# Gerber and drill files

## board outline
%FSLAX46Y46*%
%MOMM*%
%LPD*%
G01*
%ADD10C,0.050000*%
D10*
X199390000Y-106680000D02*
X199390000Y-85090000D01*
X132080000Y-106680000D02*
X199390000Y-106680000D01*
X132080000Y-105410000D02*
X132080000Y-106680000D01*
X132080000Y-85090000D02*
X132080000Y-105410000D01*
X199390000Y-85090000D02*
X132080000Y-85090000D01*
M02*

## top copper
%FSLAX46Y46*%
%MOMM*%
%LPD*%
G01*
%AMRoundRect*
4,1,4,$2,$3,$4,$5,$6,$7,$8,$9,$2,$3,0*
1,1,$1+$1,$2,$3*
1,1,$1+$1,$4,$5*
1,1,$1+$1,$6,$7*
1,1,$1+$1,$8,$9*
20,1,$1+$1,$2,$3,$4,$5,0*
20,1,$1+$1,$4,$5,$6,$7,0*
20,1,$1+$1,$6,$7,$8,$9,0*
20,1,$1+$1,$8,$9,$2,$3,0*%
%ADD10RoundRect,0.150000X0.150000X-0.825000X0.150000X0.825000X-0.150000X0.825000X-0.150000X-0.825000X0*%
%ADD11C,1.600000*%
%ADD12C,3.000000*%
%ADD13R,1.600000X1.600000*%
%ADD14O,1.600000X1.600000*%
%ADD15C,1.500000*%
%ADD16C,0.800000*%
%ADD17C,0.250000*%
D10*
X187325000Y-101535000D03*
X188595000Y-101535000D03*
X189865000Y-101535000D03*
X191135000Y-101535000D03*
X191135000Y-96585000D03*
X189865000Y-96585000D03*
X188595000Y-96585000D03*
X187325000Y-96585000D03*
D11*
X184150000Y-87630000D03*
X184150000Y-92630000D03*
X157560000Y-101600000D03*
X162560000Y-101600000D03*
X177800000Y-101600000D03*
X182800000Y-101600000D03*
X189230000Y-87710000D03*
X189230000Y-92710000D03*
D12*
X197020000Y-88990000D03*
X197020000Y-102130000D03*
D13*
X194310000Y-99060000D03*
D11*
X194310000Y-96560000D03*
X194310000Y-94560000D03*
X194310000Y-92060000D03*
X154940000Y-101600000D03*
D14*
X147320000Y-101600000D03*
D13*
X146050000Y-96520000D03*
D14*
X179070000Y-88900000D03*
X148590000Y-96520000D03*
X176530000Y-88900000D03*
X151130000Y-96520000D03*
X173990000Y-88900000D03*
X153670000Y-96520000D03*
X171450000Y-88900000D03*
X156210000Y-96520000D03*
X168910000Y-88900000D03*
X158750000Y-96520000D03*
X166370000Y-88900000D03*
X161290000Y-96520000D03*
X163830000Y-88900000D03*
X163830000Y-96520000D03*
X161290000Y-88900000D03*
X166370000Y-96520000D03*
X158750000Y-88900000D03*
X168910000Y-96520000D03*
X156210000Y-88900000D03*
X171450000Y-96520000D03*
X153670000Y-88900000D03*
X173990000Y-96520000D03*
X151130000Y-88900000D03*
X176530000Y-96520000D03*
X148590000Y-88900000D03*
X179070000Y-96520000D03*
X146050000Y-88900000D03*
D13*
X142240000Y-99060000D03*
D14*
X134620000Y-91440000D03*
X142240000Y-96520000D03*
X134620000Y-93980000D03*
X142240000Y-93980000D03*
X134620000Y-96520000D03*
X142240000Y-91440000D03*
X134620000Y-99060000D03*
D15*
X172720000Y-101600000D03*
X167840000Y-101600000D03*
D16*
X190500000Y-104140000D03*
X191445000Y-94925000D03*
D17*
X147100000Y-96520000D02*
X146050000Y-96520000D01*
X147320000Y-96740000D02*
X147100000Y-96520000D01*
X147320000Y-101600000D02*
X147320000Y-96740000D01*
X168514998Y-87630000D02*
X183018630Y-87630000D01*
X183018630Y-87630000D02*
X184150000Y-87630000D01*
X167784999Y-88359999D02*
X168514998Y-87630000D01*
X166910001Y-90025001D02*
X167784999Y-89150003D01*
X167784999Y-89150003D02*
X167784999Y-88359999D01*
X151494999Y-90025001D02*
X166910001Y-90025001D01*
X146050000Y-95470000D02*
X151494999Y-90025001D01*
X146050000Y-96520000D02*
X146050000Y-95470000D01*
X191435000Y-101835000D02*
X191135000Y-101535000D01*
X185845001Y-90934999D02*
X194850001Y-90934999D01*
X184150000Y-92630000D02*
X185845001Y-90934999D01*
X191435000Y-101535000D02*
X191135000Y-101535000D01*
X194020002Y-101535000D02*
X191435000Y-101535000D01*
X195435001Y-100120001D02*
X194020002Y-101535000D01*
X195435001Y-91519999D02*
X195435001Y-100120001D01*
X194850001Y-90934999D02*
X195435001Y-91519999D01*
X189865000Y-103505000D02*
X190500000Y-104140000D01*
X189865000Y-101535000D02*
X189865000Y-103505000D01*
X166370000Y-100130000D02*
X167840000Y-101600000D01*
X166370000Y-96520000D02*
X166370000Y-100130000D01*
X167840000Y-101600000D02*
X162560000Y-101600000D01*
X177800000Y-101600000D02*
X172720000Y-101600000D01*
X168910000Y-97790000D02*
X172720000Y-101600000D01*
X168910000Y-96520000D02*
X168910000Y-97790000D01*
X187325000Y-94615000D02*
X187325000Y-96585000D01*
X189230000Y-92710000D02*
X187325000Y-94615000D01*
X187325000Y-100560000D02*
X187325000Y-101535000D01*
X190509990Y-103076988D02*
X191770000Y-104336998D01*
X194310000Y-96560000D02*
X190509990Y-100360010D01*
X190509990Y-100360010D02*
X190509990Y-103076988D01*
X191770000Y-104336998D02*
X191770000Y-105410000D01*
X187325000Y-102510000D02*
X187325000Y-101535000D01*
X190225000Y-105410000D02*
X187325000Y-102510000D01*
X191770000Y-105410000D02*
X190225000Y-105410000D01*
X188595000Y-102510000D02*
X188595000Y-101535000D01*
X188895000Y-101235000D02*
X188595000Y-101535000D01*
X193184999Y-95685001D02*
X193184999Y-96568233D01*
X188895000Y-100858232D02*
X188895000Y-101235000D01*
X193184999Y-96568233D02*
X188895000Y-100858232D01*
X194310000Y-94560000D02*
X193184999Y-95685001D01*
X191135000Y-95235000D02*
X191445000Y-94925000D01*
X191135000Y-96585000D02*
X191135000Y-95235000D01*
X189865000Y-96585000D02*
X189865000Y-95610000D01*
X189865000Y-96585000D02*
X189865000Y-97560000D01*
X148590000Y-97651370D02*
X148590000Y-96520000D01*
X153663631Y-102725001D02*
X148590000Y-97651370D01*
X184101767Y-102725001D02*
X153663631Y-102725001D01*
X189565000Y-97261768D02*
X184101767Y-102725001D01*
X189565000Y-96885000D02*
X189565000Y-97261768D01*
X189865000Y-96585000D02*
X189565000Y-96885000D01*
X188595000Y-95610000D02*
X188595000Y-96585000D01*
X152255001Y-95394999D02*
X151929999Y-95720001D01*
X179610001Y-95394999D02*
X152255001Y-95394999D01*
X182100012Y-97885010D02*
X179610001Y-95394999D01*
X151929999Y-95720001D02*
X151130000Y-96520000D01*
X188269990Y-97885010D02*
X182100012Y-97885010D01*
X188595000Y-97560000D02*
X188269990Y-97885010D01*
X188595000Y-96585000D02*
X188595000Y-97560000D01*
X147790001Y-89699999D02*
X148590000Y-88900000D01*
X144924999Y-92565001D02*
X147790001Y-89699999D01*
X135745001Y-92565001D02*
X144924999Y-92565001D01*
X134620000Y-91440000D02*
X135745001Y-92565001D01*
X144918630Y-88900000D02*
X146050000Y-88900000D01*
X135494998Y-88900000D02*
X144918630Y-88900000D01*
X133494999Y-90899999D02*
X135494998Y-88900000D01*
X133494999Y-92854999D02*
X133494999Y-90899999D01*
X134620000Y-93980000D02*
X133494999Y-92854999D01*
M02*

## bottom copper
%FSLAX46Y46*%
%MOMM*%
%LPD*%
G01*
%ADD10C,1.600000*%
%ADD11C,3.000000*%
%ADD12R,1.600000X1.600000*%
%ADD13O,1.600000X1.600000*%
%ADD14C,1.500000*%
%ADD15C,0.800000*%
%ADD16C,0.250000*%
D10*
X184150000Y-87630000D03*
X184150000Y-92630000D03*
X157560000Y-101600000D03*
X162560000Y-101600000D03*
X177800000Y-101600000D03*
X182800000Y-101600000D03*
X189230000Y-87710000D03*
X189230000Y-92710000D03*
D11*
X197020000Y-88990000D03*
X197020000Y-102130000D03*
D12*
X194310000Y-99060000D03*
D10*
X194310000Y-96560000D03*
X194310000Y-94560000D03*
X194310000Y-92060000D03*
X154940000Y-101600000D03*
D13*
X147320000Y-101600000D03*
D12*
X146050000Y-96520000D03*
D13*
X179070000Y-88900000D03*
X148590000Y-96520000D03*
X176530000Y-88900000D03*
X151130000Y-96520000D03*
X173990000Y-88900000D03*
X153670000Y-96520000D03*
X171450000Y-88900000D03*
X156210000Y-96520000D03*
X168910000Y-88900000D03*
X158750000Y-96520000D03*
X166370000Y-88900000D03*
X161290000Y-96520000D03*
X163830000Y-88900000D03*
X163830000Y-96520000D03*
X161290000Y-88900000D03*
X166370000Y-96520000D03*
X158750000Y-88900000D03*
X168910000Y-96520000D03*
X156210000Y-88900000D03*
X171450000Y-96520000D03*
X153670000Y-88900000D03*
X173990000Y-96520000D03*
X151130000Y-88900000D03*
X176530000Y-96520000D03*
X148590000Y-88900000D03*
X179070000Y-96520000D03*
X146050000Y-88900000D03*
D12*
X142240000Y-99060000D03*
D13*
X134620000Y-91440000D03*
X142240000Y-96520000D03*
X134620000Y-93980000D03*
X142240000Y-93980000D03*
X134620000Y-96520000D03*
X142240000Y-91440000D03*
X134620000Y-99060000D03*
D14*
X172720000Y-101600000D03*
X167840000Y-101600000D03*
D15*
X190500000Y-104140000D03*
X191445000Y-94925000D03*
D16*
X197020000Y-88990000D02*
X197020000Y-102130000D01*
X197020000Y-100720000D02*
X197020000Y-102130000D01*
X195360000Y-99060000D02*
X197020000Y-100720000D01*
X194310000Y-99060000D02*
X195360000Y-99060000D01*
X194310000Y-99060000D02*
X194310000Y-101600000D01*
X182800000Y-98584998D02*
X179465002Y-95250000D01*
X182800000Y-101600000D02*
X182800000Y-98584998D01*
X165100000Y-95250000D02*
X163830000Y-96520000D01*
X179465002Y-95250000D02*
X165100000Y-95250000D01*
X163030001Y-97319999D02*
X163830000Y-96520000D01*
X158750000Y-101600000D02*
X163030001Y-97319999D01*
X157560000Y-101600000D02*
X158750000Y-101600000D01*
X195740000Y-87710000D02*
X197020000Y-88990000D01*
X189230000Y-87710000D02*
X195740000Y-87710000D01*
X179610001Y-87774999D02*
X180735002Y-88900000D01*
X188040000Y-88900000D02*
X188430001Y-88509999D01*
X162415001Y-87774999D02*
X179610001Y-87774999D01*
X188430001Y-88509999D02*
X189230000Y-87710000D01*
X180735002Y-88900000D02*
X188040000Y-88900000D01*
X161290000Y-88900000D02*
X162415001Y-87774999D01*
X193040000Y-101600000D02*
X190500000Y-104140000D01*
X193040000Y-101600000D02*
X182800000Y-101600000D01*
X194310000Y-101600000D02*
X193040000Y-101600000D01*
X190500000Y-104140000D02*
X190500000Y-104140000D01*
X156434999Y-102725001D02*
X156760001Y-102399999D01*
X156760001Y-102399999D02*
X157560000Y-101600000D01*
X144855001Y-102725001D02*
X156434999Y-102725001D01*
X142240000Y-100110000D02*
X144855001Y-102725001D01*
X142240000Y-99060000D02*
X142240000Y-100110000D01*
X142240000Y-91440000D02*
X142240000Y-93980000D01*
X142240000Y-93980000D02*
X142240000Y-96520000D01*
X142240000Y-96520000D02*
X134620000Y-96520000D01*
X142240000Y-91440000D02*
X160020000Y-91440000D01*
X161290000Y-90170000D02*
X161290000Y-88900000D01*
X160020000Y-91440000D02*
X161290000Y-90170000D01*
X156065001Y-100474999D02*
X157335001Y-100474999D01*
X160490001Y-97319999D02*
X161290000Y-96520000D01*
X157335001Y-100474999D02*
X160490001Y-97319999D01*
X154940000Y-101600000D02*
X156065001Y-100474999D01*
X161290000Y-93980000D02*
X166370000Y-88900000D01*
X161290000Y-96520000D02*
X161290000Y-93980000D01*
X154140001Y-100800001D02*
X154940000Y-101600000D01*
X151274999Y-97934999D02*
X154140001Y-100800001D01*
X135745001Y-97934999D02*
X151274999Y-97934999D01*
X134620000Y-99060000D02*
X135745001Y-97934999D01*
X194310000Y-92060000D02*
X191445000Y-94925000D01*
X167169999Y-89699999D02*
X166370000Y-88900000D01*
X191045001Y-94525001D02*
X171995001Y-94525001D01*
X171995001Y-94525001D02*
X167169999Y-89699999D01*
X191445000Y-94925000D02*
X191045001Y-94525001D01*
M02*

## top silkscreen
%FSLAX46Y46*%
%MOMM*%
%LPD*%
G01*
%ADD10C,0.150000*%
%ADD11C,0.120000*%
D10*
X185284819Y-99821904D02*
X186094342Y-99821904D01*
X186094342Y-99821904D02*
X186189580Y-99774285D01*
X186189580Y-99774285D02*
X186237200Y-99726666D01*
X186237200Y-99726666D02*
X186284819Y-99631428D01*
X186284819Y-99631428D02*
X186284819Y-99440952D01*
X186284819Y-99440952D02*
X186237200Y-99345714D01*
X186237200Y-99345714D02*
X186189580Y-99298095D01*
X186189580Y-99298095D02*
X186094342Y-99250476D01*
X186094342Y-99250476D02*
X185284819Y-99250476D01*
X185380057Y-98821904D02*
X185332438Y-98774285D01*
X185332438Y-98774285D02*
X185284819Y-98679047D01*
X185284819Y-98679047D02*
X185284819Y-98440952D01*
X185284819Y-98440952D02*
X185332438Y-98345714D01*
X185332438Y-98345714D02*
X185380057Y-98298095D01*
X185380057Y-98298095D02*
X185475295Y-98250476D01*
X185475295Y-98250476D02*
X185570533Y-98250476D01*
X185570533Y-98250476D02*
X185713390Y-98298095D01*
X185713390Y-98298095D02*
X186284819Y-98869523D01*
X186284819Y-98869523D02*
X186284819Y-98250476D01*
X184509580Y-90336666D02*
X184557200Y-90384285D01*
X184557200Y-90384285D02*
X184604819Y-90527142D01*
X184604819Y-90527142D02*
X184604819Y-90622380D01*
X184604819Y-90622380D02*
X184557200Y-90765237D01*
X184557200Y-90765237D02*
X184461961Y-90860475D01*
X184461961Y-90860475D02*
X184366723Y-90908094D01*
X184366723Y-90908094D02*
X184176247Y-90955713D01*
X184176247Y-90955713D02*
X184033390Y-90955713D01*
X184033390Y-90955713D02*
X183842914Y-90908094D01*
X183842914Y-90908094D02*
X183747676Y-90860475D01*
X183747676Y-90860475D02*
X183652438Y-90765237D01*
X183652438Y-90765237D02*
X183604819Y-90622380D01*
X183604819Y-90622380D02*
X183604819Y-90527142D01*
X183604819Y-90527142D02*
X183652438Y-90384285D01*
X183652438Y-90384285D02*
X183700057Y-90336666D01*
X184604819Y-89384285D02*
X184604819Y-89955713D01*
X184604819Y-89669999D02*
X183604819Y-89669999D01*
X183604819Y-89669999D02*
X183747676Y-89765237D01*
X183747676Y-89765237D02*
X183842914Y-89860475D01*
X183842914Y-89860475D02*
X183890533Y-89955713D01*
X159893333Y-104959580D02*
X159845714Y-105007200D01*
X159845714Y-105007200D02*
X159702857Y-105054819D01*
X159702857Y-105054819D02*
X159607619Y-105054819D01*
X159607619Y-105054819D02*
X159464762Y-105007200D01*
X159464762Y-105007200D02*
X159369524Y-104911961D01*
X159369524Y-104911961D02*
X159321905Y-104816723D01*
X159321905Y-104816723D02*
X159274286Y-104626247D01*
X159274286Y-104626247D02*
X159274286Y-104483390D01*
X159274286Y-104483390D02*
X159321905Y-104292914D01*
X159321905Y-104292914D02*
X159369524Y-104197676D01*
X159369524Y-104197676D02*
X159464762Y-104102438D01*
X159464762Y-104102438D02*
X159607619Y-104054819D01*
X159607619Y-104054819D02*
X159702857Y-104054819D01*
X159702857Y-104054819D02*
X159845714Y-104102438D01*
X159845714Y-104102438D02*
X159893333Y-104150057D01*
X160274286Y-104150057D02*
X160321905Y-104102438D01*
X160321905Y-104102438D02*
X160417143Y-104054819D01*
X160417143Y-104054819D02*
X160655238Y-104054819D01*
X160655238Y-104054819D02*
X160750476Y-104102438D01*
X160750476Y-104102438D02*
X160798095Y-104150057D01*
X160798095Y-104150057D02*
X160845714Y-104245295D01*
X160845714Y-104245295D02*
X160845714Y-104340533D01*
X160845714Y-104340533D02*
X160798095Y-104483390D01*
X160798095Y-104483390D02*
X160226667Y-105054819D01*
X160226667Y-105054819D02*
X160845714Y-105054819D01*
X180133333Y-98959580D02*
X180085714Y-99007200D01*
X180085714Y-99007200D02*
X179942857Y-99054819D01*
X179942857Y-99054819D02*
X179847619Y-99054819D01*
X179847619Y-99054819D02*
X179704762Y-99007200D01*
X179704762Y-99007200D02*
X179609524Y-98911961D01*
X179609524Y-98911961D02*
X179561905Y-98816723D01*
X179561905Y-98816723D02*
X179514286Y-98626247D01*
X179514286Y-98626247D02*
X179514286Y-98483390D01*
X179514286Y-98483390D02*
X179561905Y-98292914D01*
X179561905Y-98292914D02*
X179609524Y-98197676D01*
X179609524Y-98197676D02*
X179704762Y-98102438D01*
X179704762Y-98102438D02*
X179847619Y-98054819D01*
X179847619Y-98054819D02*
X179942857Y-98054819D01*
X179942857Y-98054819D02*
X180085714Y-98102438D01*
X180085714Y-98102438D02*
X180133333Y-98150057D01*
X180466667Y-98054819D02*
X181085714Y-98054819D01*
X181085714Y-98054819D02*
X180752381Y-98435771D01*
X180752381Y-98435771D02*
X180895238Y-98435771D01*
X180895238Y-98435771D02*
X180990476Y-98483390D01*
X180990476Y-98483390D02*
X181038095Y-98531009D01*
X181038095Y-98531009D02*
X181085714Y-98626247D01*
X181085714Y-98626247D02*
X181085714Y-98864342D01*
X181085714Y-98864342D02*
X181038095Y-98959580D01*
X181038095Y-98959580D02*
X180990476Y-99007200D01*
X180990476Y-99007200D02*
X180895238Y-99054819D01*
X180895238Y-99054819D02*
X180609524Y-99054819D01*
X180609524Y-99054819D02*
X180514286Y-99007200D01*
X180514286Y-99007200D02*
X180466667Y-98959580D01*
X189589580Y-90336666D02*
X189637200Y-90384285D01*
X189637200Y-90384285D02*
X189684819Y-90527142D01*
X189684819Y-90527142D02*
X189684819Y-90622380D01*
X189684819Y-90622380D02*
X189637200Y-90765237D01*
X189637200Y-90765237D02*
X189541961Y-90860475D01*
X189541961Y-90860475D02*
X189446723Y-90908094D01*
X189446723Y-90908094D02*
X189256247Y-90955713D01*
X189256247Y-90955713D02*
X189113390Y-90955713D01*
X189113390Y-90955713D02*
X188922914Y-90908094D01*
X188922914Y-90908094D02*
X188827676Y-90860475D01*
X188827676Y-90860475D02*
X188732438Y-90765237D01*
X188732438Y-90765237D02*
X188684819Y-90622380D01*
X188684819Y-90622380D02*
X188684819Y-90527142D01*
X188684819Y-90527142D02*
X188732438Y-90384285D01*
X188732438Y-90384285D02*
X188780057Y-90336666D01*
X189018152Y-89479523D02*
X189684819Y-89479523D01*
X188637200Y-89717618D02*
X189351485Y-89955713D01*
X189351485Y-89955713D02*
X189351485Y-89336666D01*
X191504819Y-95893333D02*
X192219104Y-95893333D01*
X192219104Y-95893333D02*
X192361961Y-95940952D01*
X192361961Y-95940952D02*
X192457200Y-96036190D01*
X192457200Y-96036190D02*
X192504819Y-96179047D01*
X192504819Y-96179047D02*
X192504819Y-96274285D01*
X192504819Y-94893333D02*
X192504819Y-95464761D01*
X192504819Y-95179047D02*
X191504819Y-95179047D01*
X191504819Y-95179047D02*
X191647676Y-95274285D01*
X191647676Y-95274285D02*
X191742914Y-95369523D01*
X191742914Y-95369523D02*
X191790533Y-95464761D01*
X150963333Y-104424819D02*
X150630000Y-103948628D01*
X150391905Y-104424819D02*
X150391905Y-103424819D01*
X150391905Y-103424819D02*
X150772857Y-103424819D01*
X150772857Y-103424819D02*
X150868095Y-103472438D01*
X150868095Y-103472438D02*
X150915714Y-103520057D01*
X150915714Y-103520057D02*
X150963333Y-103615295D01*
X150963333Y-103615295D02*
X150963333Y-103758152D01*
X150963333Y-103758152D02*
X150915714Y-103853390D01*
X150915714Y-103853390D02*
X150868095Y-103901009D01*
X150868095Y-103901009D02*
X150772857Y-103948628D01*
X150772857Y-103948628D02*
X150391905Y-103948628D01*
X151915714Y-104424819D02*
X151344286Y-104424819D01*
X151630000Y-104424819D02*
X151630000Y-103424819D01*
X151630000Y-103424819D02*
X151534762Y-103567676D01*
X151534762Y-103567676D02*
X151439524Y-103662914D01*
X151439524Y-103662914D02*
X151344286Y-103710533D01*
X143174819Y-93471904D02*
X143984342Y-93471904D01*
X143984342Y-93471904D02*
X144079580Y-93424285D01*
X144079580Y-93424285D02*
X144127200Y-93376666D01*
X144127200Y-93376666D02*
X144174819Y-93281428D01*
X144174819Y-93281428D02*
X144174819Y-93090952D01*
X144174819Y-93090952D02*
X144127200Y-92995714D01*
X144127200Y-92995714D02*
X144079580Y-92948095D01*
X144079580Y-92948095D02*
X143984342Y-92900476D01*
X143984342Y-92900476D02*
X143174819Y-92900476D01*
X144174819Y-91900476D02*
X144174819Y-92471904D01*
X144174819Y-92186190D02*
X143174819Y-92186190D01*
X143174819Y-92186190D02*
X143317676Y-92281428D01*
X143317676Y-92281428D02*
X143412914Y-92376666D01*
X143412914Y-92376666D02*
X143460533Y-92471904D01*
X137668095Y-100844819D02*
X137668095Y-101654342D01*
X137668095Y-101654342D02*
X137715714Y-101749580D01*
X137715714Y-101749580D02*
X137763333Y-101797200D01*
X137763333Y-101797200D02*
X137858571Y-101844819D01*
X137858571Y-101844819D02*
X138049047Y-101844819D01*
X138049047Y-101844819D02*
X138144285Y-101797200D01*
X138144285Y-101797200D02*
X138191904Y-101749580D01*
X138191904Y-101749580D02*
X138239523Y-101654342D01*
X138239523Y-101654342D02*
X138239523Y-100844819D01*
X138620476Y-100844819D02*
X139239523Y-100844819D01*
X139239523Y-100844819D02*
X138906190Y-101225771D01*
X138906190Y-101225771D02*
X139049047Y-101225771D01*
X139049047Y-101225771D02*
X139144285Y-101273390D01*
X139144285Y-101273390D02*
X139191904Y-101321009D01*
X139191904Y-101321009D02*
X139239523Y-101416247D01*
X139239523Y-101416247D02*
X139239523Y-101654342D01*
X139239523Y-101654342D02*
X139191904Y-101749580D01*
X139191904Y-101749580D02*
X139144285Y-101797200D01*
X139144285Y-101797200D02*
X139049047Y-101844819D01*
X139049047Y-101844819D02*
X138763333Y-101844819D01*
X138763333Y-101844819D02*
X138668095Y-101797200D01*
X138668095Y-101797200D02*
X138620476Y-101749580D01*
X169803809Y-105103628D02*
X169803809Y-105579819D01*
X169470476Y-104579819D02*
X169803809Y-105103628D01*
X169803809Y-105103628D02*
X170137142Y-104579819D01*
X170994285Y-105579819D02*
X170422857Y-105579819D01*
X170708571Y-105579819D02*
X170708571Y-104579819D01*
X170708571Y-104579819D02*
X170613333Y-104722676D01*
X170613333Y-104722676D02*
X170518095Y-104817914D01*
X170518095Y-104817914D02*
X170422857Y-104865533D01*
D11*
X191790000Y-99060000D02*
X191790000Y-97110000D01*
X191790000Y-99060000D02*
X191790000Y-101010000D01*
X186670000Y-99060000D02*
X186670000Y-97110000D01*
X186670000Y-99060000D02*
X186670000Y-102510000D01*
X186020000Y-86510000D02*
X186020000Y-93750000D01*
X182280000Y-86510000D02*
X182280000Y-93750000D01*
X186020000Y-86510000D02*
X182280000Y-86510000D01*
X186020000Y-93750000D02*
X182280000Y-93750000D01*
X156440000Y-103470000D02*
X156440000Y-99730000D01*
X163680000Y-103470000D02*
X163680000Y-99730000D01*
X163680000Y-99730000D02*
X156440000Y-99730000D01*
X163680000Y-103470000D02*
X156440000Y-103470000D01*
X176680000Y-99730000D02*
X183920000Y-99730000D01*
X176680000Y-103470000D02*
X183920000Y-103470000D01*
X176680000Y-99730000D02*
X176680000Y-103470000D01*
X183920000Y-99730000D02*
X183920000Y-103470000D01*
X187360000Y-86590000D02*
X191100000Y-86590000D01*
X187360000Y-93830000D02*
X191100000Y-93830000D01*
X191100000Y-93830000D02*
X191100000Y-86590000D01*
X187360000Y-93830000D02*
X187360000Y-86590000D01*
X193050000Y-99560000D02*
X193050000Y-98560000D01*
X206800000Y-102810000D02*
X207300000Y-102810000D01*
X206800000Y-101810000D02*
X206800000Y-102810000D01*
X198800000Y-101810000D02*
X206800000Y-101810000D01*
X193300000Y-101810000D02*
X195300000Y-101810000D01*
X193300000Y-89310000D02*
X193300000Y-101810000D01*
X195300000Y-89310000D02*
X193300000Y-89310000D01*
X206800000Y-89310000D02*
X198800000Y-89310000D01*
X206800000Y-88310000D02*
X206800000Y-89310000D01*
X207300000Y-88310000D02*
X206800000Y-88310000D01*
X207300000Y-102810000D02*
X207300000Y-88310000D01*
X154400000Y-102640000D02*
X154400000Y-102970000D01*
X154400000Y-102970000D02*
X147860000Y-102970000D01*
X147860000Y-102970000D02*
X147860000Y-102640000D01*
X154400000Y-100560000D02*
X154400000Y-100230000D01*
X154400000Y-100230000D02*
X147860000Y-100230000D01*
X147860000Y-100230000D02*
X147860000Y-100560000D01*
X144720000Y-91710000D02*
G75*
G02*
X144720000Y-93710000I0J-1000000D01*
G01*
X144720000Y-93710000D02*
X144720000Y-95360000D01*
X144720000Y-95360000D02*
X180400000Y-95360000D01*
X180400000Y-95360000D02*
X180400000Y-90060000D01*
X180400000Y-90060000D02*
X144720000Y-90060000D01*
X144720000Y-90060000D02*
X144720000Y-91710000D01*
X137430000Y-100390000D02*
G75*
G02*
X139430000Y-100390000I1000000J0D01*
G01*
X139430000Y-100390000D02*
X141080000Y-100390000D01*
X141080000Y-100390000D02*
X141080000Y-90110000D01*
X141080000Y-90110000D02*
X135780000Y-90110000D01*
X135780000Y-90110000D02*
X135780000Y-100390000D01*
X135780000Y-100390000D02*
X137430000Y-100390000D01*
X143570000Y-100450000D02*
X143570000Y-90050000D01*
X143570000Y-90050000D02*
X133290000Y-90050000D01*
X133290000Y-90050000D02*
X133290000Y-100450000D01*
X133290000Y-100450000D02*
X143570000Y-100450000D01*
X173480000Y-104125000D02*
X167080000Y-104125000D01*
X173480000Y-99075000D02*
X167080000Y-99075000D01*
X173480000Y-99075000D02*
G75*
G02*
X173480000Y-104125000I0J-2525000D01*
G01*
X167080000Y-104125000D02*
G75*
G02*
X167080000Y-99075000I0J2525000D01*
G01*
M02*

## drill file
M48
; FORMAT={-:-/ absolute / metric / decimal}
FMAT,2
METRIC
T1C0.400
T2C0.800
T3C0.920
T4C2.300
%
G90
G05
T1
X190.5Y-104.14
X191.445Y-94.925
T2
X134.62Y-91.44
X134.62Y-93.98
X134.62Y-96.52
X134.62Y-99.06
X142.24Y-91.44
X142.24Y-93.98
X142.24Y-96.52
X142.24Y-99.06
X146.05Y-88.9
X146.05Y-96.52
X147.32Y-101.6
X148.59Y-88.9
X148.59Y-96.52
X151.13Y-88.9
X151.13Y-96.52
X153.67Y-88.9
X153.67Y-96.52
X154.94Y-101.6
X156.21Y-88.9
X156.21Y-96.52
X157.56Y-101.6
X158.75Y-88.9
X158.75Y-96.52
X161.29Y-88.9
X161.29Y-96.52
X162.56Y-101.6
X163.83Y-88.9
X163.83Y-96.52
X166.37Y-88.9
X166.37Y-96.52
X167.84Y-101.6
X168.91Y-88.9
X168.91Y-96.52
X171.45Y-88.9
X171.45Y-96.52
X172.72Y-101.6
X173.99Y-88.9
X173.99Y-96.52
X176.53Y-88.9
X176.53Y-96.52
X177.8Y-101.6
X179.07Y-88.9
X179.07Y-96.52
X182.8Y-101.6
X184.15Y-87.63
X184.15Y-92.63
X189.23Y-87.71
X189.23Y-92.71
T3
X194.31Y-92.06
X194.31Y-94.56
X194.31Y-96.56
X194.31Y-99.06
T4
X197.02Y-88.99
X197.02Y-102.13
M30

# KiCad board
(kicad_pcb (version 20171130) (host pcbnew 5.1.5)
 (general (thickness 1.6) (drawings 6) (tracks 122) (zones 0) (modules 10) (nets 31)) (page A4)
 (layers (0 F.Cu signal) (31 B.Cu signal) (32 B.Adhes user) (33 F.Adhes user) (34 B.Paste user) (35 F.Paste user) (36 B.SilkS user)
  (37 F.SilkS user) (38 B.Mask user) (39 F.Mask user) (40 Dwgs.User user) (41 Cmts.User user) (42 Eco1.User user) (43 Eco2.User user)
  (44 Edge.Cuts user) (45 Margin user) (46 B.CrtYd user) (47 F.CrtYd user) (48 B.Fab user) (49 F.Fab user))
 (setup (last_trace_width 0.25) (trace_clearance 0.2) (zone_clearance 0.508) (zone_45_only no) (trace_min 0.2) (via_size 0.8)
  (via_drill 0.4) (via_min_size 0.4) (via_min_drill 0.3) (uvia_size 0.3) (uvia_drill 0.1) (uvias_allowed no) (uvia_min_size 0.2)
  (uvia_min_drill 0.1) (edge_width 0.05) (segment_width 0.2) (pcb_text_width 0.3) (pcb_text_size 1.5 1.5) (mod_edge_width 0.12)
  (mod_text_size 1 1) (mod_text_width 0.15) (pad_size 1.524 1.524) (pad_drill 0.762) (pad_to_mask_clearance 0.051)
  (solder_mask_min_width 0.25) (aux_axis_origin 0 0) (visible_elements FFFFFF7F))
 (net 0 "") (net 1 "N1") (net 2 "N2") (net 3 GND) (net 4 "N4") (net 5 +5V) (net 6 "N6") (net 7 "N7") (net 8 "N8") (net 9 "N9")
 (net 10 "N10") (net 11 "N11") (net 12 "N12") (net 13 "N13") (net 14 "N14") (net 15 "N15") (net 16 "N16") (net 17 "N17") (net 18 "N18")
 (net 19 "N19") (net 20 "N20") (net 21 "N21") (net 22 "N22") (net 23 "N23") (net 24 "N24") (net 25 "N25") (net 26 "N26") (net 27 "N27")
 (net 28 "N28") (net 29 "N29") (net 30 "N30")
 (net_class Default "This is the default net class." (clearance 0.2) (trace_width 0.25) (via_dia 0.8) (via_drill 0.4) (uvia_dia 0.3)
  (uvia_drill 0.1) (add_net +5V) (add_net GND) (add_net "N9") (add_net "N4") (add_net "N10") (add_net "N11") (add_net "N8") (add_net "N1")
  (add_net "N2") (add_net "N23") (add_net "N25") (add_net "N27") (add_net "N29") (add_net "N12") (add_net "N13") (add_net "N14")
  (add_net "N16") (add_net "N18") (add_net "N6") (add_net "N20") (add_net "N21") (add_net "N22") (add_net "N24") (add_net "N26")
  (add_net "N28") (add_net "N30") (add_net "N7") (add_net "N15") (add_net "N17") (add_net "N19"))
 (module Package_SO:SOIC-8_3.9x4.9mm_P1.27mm (layer F.Cu) (at 189.23 99.06 90)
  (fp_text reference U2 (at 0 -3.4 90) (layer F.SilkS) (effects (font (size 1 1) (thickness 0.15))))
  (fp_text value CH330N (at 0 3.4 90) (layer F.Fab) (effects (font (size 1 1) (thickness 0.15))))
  (fp_line (start 0 2.56) (end 1.95 2.56) (layer F.SilkS) (width 0.12))
  (fp_line (start 0 2.56) (end -1.95 2.56) (layer F.SilkS) (width 0.12))
  (fp_line (start 0 -2.56) (end 1.95 -2.56) (layer F.SilkS) (width 0.12))
  (fp_line (start 0 -2.56) (end -3.45 -2.56) (layer F.SilkS) (width 0.12))
  (pad 1 smd roundrect (at -2.475 -1.905 90) (size 1.95 0.6) (layers F.Cu F.Paste F.Mask) (roundrect_rratio 0.25) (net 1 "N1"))
  (pad 2 smd roundrect (at -2.475 -0.635 90) (size 1.95 0.6) (layers F.Cu F.Paste F.Mask) (roundrect_rratio 0.25) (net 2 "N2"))
  (pad 3 smd roundrect (at -2.475 0.635 90) (size 1.95 0.6) (layers F.Cu F.Paste F.Mask) (roundrect_rratio 0.25) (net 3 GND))
  (pad 4 smd roundrect (at -2.475 1.905 90) (size 1.95 0.6) (layers F.Cu F.Paste F.Mask) (roundrect_rratio 0.25) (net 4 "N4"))
  (pad 5 smd roundrect (at 2.475 1.905 90) (size 1.95 0.6) (layers F.Cu F.Paste F.Mask) (roundrect_rratio 0.25) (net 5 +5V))
  (pad 6 smd roundrect (at 2.475 0.635 90) (size 1.95 0.6) (layers F.Cu F.Paste F.Mask) (roundrect_rratio 0.25) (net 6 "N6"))
  (pad 7 smd roundrect (at 2.475 -0.635 90) (size 1.95 0.6) (layers F.Cu F.Paste F.Mask) (roundrect_rratio 0.25) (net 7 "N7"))
  (pad 8 smd roundrect (at 2.475 -1.905 90) (size 1.95 0.6) (layers F.Cu F.Paste F.Mask) (roundrect_rratio 0.25) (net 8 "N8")))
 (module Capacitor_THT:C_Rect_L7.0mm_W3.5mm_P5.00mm (layer F.Cu) (at 184.15 87.63 270)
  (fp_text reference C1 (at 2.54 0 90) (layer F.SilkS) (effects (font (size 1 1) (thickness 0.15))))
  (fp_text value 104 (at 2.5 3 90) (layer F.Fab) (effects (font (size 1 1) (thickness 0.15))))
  (fp_line (start -1.12 -1.87) (end 6.12 -1.87) (layer F.SilkS) (width 0.12))
  (fp_line (start -1.12 1.87) (end 6.12 1.87) (layer F.SilkS) (width 0.12))
  (fp_line (start -1.12 -1.87) (end -1.12 1.87) (layer F.SilkS) (width 0.12))
  (fp_line (start 6.12 -1.87) (end 6.12 1.87) (layer F.SilkS) (width 0.12))
  (pad 1 thru_hole circle (at 0 0 270) (size 1.6 1.6) (drill 0.8) (layers *.Cu *.Mask) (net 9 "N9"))
  (pad 2 thru_hole circle (at 5 0 270) (size 1.6 1.6) (drill 0.8) (layers *.Cu *.Mask) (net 4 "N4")))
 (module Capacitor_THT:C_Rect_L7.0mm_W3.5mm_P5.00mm (layer F.Cu) (at 162.56 101.6 180)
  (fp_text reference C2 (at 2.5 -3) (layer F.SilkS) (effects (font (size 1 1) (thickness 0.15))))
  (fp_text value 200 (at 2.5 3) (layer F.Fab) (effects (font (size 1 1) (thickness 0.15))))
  (fp_line (start 6.12 -1.87) (end 6.12 1.87) (layer F.SilkS) (width 0.12))
  (fp_line (start -1.12 -1.87) (end -1.12 1.87) (layer F.SilkS) (width 0.12))
  (fp_line (start -1.12 1.87) (end 6.12 1.87) (layer F.SilkS) (width 0.12))
  (fp_line (start -1.12 -1.87) (end 6.12 -1.87) (layer F.SilkS) (width 0.12))
  (pad 2 thru_hole circle (at 5 0 180) (size 1.6 1.6) (drill 0.8) (layers *.Cu *.Mask) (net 3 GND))
  (pad 1 thru_hole circle (at 0 0 180) (size 1.6 1.6) (drill 0.8) (layers *.Cu *.Mask) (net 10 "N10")))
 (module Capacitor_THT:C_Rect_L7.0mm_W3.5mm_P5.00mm (layer F.Cu) (at 177.8 101.6)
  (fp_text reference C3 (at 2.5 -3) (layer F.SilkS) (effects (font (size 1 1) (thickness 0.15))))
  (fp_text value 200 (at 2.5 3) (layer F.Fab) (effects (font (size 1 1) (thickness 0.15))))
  (fp_line (start -1.12 -1.87) (end 6.12 -1.87) (layer F.SilkS) (width 0.12))
  (fp_line (start -1.12 1.87) (end 6.12 1.87) (layer F.SilkS) (width 0.12))
  (fp_line (start -1.12 -1.87) (end -1.12 1.87) (layer F.SilkS) (width 0.12))
  (fp_line (start 6.12 -1.87) (end 6.12 1.87) (layer F.SilkS) (width 0.12))
  (pad 1 thru_hole circle (at 0 0) (size 1.6 1.6) (drill 0.8) (layers *.Cu *.Mask) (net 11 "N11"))
  (pad 2 thru_hole circle (at 5 0) (size 1.6 1.6) (drill 0.8) (layers *.Cu *.Mask) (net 3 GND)))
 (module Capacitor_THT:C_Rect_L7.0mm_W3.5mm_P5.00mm (layer F.Cu) (at 189.23 92.71 90)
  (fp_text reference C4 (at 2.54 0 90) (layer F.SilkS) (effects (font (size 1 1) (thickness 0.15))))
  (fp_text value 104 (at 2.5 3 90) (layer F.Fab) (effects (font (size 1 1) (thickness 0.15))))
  (fp_line (start 6.12 -1.87) (end 6.12 1.87) (layer F.SilkS) (width 0.12))
  (fp_line (start -1.12 -1.87) (end -1.12 1.87) (layer F.SilkS) (width 0.12))
  (fp_line (start -1.12 1.87) (end 6.12 1.87) (layer F.SilkS) (width 0.12))
  (fp_line (start -1.12 -1.87) (end 6.12 -1.87) (layer F.SilkS) (width 0.12))
  (pad 2 thru_hole circle (at 5 0 90) (size 1.6 1.6) (drill 0.8) (layers *.Cu *.Mask) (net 3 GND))
  (pad 1 thru_hole circle (at 0 0 90) (size 1.6 1.6) (drill 0.8) (layers *.Cu *.Mask) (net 8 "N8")))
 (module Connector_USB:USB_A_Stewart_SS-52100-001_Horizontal (layer F.Cu) (at 194.31 99.06 90)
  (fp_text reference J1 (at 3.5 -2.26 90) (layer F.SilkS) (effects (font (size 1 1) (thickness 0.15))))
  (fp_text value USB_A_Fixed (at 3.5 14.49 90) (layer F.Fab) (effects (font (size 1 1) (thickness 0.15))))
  (fp_line (start -0.5 -1.26) (end 0.5 -1.26) (layer F.SilkS) (width 0.12))
  (fp_line (start -3.75 12.49) (end -3.75 12.99) (layer F.SilkS) (width 0.12))
  (fp_line (start -2.75 12.49) (end -3.75 12.49) (layer F.SilkS) (width 0.12))
  (fp_line (start -2.75 4.49) (end -2.75 12.49) (layer F.SilkS) (width 0.12))
  (fp_line (start -2.75 -1.01) (end -2.75 0.99) (layer F.SilkS) (width 0.12))
  (fp_line (start 9.75 -1.01) (end -2.75 -1.01) (layer F.SilkS) (width 0.12))
  (fp_line (start 9.75 0.99) (end 9.75 -1.01) (layer F.SilkS) (width 0.12))
  (fp_line (start 9.75 12.49) (end 9.75 4.49) (layer F.SilkS) (width 0.12))
  (fp_line (start 10.75 12.49) (end 9.75 12.49) (layer F.SilkS) (width 0.12))
  (fp_line (start 10.75 12.99) (end 10.75 12.49) (layer F.SilkS) (width 0.12))
  (fp_line (start -3.75 12.99) (end 10.75 12.99) (layer F.SilkS) (width 0.12))
  (pad 5 thru_hole circle (at 10.07 2.71 90) (size 3 3) (drill 2.3) (layers *.Cu *.Mask) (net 3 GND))
  (pad 5 thru_hole circle (at -3.07 2.71 90) (size 3 3) (drill 2.3) (layers *.Cu *.Mask) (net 3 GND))
  (pad 1 thru_hole rect (at 0 0 90) (size 1.6 1.6) (drill 0.92) (layers *.Cu *.Mask) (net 3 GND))
  (pad 2 thru_hole circle (at 2.5 0 90) (size 1.6 1.6) (drill 0.92) (layers *.Cu *.Mask) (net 1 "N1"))
  (pad 3 thru_hole circle (at 4.5 0 90) (size 1.6 1.6) (drill 0.92) (layers *.Cu *.Mask) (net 2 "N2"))
  (pad 4 thru_hole circle (at 7 0 90) (size 1.6 1.6) (drill 0.92) (layers *.Cu *.Mask) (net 5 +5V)))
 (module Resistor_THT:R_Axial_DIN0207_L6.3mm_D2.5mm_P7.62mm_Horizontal (layer F.Cu) (at 154.94 101.6 180)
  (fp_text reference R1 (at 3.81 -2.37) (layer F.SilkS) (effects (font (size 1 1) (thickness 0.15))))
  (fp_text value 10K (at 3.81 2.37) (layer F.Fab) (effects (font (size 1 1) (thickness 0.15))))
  (fp_line (start 0.54 -1.04) (end 0.54 -1.37) (layer F.SilkS) (width 0.12))
  (fp_line (start 0.54 -1.37) (end 7.08 -1.37) (layer F.SilkS) (width 0.12))
  (fp_line (start 7.08 -1.37) (end 7.08 -1.04) (layer F.SilkS) (width 0.12))
  (fp_line (start 0.54 1.04) (end 0.54 1.37) (layer F.SilkS) (width 0.12))
  (fp_line (start 0.54 1.37) (end 7.08 1.37) (layer F.SilkS) (width 0.12))
  (fp_line (start 7.08 1.37) (end 7.08 1.04) (layer F.SilkS) (width 0.12))
  (pad 1 thru_hole circle (at 0 0 180) (size 1.6 1.6) (drill 0.8) (layers *.Cu *.Mask) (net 5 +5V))
  (pad 2 thru_hole oval (at 7.62 0 180) (size 1.6 1.6) (drill 0.8) (layers *.Cu *.Mask) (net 9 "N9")))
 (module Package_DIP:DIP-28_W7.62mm (layer F.Cu) (at 146.05 96.52 90)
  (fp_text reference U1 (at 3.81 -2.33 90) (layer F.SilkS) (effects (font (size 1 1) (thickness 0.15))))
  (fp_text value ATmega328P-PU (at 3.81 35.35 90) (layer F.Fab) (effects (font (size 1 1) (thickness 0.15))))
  (fp_arc (start 3.81 -1.33) (end 2.81 -1.33) (angle -180) (layer F.SilkS) (width 0.12))
  (fp_line (start 2.81 -1.33) (end 1.16 -1.33) (layer F.SilkS) (width 0.12))
  (fp_line (start 1.16 -1.33) (end 1.16 34.35) (layer F.SilkS) (width 0.12))
  (fp_line (start 1.16 34.35) (end 6.46 34.35) (layer F.SilkS) (width 0.12))
  (fp_line (start 6.46 34.35) (end 6.46 -1.33) (layer F.SilkS) (width 0.12))
  (fp_line (start 6.46 -1.33) (end 4.81 -1.33) (layer F.SilkS) (width 0.12))
  (pad 1 thru_hole rect (at 0 0 90) (size 1.6 1.6) (drill 0.8) (layers *.Cu *.Mask) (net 9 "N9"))
  (pad 15 thru_hole oval (at 7.62 33.02 90) (size 1.6 1.6) (drill 0.8) (layers *.Cu *.Mask) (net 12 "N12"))
  (pad 2 thru_hole oval (at 0 2.54 90) (size 1.6 1.6) (drill 0.8) (layers *.Cu *.Mask) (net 6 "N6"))
  (pad 16 thru_hole oval (at 7.62 30.48 90) (size 1.6 1.6) (drill 0.8) (layers *.Cu *.Mask) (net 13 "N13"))
  (pad 3 thru_hole oval (at 0 5.08 90) (size 1.6 1.6) (drill 0.8) (layers *.Cu *.Mask) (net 7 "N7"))
  (pad 17 thru_hole oval (at 7.62 27.94 90) (size 1.6 1.6) (drill 0.8) (layers *.Cu *.Mask) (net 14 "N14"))
  (pad 4 thru_hole oval (at 0 7.62 90) (size 1.6 1.6) (drill 0.8) (layers *.Cu *.Mask) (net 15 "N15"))
  (pad 18 thru_hole oval (at 7.62 25.4 90) (size 1.6 1.6) (drill 0.8) (layers *.Cu *.Mask) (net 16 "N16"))
  (pad 5 thru_hole oval (at 0 10.16 90) (size 1.6 1.6) (drill 0.8) (layers *.Cu *.Mask) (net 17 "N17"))
  (pad 19 thru_hole oval (at 7.62 22.86 90) (size 1.6 1.6) (drill 0.8) (layers *.Cu *.Mask) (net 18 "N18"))
  (pad 6 thru_hole oval (at 0 12.7 90) (size 1.6 1.6) (drill 0.8) (layers *.Cu *.Mask) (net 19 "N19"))
  (pad 20 thru_hole oval (at 7.62 20.32 90) (size 1.6 1.6) (drill 0.8) (layers *.Cu *.Mask) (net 5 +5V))
  (pad 7 thru_hole oval (at 0 15.24 90) (size 1.6 1.6) (drill 0.8) (layers *.Cu *.Mask) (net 5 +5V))
  (pad 21 thru_hole oval (at 7.62 17.78 90) (size 1.6 1.6) (drill 0.8) (layers *.Cu *.Mask) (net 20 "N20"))
  (pad 8 thru_hole oval (at 0 17.78 90) (size 1.6 1.6) (drill 0.8) (layers *.Cu *.Mask) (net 3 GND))
  (pad 22 thru_hole oval (at 7.62 15.24 90) (size 1.6 1.6) (drill 0.8) (layers *.Cu *.Mask) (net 3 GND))
  (pad 9 thru_hole oval (at 0 20.32 90) (size 1.6 1.6) (drill 0.8) (layers *.Cu *.Mask) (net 10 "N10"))
  (pad 23 thru_hole oval (at 7.62 12.7 90) (size 1.6 1.6) (drill 0.8) (layers *.Cu *.Mask) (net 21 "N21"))
  (pad 10 thru_hole oval (at 0 22.86 90) (size 1.6 1.6) (drill 0.8) (layers *.Cu *.Mask) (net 11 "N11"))
  (pad 24 thru_hole oval (at 7.62 10.16 90) (size 1.6 1.6) (drill 0.8) (layers *.Cu *.Mask) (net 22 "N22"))
  (pad 11 thru_hole oval (at 0 25.4 90) (size 1.6 1.6) (drill 0.8) (layers *.Cu *.Mask) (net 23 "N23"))
  (pad 25 thru_hole oval (at 7.62 7.62 90) (size 1.6 1.6) (drill 0.8) (layers *.Cu *.Mask) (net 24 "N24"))
  (pad 12 thru_hole oval (at 0 27.94 90) (size 1.6 1.6) (drill 0.8) (layers *.Cu *.Mask) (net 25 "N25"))
  (pad 26 thru_hole oval (at 7.62 5.08 90) (size 1.6 1.6) (drill 0.8) (layers *.Cu *.Mask) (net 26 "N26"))
  (pad 13 thru_hole oval (at 0 30.48 90) (size 1.6 1.6) (drill 0.8) (layers *.Cu *.Mask) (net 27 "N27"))
  (pad 27 thru_hole oval (at 7.62 2.54 90) (size 1.6 1.6) (drill 0.8) (layers *.Cu *.Mask) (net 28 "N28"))
  (pad 14 thru_hole oval (at 0 33.02 90) (size 1.6 1.6) (drill 0.8) (layers *.Cu *.Mask) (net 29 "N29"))
  (pad 28 thru_hole oval (at 7.62 0 90) (size 1.6 1.6) (drill 0.8) (layers *.Cu *.Mask) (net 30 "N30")))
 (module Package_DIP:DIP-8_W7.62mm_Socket (layer F.Cu) (at 142.24 99.06 180)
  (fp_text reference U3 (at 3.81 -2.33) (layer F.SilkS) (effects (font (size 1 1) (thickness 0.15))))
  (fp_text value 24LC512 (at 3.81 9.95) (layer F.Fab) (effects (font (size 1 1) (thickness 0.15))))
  (fp_arc (start 3.81 -1.33) (end 2.81 -1.33) (angle -180) (layer F.SilkS) (width 0.12))
  (fp_line (start 2.81 -1.33) (end 1.16 -1.33) (layer F.SilkS) (width 0.12))
  (fp_line (start 1.16 -1.33) (end 1.16 8.95) (layer F.SilkS) (width 0.12))
  (fp_line (start 1.16 8.95) (end 6.46 8.95) (layer F.SilkS) (width 0.12))
  (fp_line (start 6.46 8.95) (end 6.46 -1.33) (layer F.SilkS) (width 0.12))
  (fp_line (start 6.46 -1.33) (end 4.81 -1.33) (layer F.SilkS) (width 0.12))
  (fp_line (start -1.33 -1.39) (end -1.33 9.01) (layer F.SilkS) (width 0.12))
  (fp_line (start -1.33 9.01) (end 8.95 9.01) (layer F.SilkS) (width 0.12))
  (fp_line (start 8.95 9.01) (end 8.95 -1.39) (layer F.SilkS) (width 0.12))
  (fp_line (start 8.95 -1.39) (end -1.33 -1.39) (layer F.SilkS) (width 0.12))
  (pad 1 thru_hole rect (at 0 0 180) (size 1.6 1.6) (drill 0.8) (layers *.Cu *.Mask) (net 3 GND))
  (pad 5 thru_hole oval (at 7.62 7.62 180) (size 1.6 1.6) (drill 0.8) (layers *.Cu *.Mask) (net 28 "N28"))
  (pad 2 thru_hole oval (at 0 2.54 180) (size 1.6 1.6) (drill 0.8) (layers *.Cu *.Mask) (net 3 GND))
  (pad 6 thru_hole oval (at 7.62 5.08 180) (size 1.6 1.6) (drill 0.8) (layers *.Cu *.Mask) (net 30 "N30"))
  (pad 3 thru_hole oval (at 0 5.08 180) (size 1.6 1.6) (drill 0.8) (layers *.Cu *.Mask) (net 3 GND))
  (pad 7 thru_hole oval (at 7.62 2.54 180) (size 1.6 1.6) (drill 0.8) (layers *.Cu *.Mask) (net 3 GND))
  (pad 4 thru_hole oval (at 0 7.62 180) (size 1.6 1.6) (drill 0.8) (layers *.Cu *.Mask) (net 3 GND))
  (pad 8 thru_hole oval (at 7.62 0 180) (size 1.6 1.6) (drill 0.8) (layers *.Cu *.Mask) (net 5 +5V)))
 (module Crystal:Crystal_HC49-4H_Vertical (layer F.Cu) (at 172.72 101.6 180)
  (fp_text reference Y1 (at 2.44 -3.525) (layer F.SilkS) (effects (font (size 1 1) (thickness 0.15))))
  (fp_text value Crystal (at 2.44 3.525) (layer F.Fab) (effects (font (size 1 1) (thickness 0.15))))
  (fp_line (start -0.76 -2.525) (end 5.64 -2.525) (layer F.SilkS) (width 0.12))
  (fp_line (start -0.76 2.525) (end 5.64 2.525) (layer F.SilkS) (width 0.12))
  (fp_arc (start -0.76 0) (end -0.76 -2.525) (angle -180) (layer F.SilkS) (width 0.12))
  (fp_arc (start 5.64 0) (end 5.64 -2.525) (angle 180) (layer F.SilkS) (width 0.12))
  (pad 1 thru_hole circle (at 0 0 180) (size 1.5 1.5) (drill 0.8) (layers *.Cu *.Mask) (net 11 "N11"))
  (pad 2 thru_hole circle (at 4.88 0 180) (size 1.5 1.5) (drill 0.8) (layers *.Cu *.Mask) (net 10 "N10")))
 (gr_line (start 199.39 106.68) (end 199.39 85.09) (layer Edge.Cuts) (width 0.05))
 (gr_line (start 132.08 106.68) (end 199.39 106.68) (layer Edge.Cuts) (width 0.05))
 (gr_line (start 132.08 105.41) (end 132.08 106.68) (layer Edge.Cuts) (width 0.05))
 (gr_line (start 132.08 85.09) (end 132.08 105.41) (layer Edge.Cuts) (width 0.05))
 (gr_line (start 199.39 85.09) (end 132.08 85.09) (layer Edge.Cuts) (width 0.05))
 (segment (start 147.1 96.52) (end 146.05 96.52) (width 0.25) (layer F.Cu) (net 9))
 (segment (start 147.32 96.74) (end 147.1 96.52) (width 0.25) (layer F.Cu) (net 9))
 (segment (start 147.32 101.6) (end 147.32 96.74) (width 0.25) (layer F.Cu) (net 9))
 (segment (start 168.514998 87.63) (end 183.01863 87.63) (width 0.25) (layer F.Cu) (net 9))
 (segment (start 183.01863 87.63) (end 184.15 87.63) (width 0.25) (layer F.Cu) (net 9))
 (segment (start 167.784999 88.359999) (end 168.514998 87.63) (width 0.25) (layer F.Cu) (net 9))
 (segment (start 166.910001 90.025001) (end 167.784999 89.150003) (width 0.25) (layer F.Cu) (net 9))
 (segment (start 167.784999 89.150003) (end 167.784999 88.359999) (width 0.25) (layer F.Cu) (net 9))
 (segment (start 151.494999 90.025001) (end 166.910001 90.025001) (width 0.25) (layer F.Cu) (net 9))
 (segment (start 146.05 95.47) (end 151.494999 90.025001) (width 0.25) (layer F.Cu) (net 9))
 (segment (start 146.05 96.52) (end 146.05 95.47) (width 0.25) (layer F.Cu) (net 9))
 (segment (start 191.435 101.835) (end 191.135 101.535) (width 0.25) (layer F.Cu) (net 4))
 (segment (start 185.845001 90.934999) (end 194.850001 90.934999) (width 0.25) (layer F.Cu) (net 4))
 (segment (start 184.15 92.63) (end 185.845001 90.934999) (width 0.25) (layer F.Cu) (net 4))
 (segment (start 191.435 101.535) (end 191.135 101.535) (width 0.25) (layer F.Cu) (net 4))
 (segment (start 194.020002 101.535) (end 191.435 101.535) (width 0.25) (layer F.Cu) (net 4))
 (segment (start 195.435001 100.120001) (end 194.020002 101.535) (width 0.25) (layer F.Cu) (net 4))
 (segment (start 195.435001 91.519999) (end 195.435001 100.120001) (width 0.25) (layer F.Cu) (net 4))
 (segment (start 194.850001 90.934999) (end 195.435001 91.519999) (width 0.25) (layer F.Cu) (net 4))
 (segment (start 197.02 88.99) (end 197.02 102.13) (width 0.25) (layer B.Cu) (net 3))
 (segment (start 197.02 100.72) (end 197.02 102.13) (width 0.25) (layer B.Cu) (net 3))
 (segment (start 195.36 99.06) (end 197.02 100.72) (width 0.25) (layer B.Cu) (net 3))
 (segment (start 194.31 99.06) (end 195.36 99.06) (width 0.25) (layer B.Cu) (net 3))
 (segment (start 194.31 99.06) (end 194.31 101.6) (width 0.25) (layer B.Cu) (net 3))
 (segment (start 182.8 98.584998) (end 179.465002 95.25) (width 0.25) (layer B.Cu) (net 3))
 (segment (start 182.8 101.6) (end 182.8 98.584998) (width 0.25) (layer B.Cu) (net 3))
 (segment (start 165.1 95.25) (end 163.83 96.52) (width 0.25) (layer B.Cu) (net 3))
 (segment (start 179.465002 95.25) (end 165.1 95.25) (width 0.25) (layer B.Cu) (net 3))
 (segment (start 163.030001 97.319999) (end 163.83 96.52) (width 0.25) (layer B.Cu) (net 3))
 (segment (start 158.75 101.6) (end 163.030001 97.319999) (width 0.25) (layer B.Cu) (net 3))
 (segment (start 157.56 101.6) (end 158.75 101.6) (width 0.25) (layer B.Cu) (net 3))
 (segment (start 195.74 87.71) (end 197.02 88.99) (width 0.25) (layer B.Cu) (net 3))
 (segment (start 189.23 87.71) (end 195.74 87.71) (width 0.25) (layer B.Cu) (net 3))
 (segment (start 179.610001 87.774999) (end 180.735002 88.9) (width 0.25) (layer B.Cu) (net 3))
 (segment (start 188.04 88.9) (end 188.430001 88.509999) (width 0.25) (layer B.Cu) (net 3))
 (segment (start 162.415001 87.774999) (end 179.610001 87.774999) (width 0.25) (layer B.Cu) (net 3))
 (segment (start 188.430001 88.509999) (end 189.23 87.71) (width 0.25) (layer B.Cu) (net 3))
 (segment (start 180.735002 88.9) (end 188.04 88.9) (width 0.25) (layer B.Cu) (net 3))
 (segment (start 161.29 88.9) (end 162.415001 87.774999) (width 0.25) (layer B.Cu) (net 3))
 (segment (start 193.04 101.6) (end 190.5 104.14) (width 0.25) (layer B.Cu) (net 3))
 (segment (start 193.04 101.6) (end 182.8 101.6) (width 0.25) (layer B.Cu) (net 3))
 (segment (start 194.31 101.6) (end 193.04 101.6) (width 0.25) (layer B.Cu) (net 3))
 (segment (start 190.5 104.14) (end 190.5 104.14) (width 0.25) (layer B.Cu) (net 3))
 (via (at 190.5 104.14) (size 0.8) (drill 0.4) (layers F.Cu B.Cu) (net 3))
 (segment (start 156.434999 102.725001) (end 156.760001 102.399999) (width 0.25) (layer B.Cu) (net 3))
 (segment (start 156.760001 102.399999) (end 157.56 101.6) (width 0.25) (layer B.Cu) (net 3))
 (segment (start 144.855001 102.725001) (end 156.434999 102.725001) (width 0.25) (layer B.Cu) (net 3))
 (segment (start 142.24 100.11) (end 144.855001 102.725001) (width 0.25) (layer B.Cu) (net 3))
 (segment (start 142.24 99.06) (end 142.24 100.11) (width 0.25) (layer B.Cu) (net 3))
 (segment (start 142.24 91.44) (end 142.24 93.98) (width 0.25) (layer B.Cu) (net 3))
 (segment (start 142.24 93.98) (end 142.24 96.52) (width 0.25) (layer B.Cu) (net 3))
 (segment (start 142.24 96.52) (end 134.62 96.52) (width 0.25) (layer B.Cu) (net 3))
 (segment (start 142.24 91.44) (end 160.02 91.44) (width 0.25) (layer B.Cu) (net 3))
 (segment (start 161.29 90.17) (end 161.29 88.9) (width 0.25) (layer B.Cu) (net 3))
 (segment (start 160.02 91.44) (end 161.29 90.17) (width 0.25) (layer B.Cu) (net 3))
 (segment (start 189.865 103.505) (end 190.5 104.14) (width 0.25) (layer F.Cu) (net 3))
 (segment (start 189.865 101.535) (end 189.865 103.505) (width 0.25) (layer F.Cu) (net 3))
 (segment (start 166.37 100.13) (end 167.84 101.6) (width 0.25) (layer F.Cu) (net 10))
 (segment (start 166.37 96.52) (end 166.37 100.13) (width 0.25) (layer F.Cu) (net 10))
 (segment (start 167.84 101.6) (end 162.56 101.6) (width 0.25) (layer F.Cu) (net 10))
 (segment (start 177.8 101.6) (end 172.72 101.6) (width 0.25) (layer F.Cu) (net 11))
 (segment (start 168.91 97.79) (end 172.72 101.6) (width 0.25) (layer F.Cu) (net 11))
 (segment (start 168.91 96.52) (end 168.91 97.79) (width 0.25) (layer F.Cu) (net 11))
 (segment (start 187.325 94.615) (end 187.325 96.585) (width 0.25) (layer F.Cu) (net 8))
 (segment (start 189.23 92.71) (end 187.325 94.615) (width 0.25) (layer F.Cu) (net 8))
 (segment (start 187.325 100.56) (end 187.325 101.535) (width 0.25) (layer F.Cu) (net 1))
 (segment (start 190.50999 103.076988) (end 191.77 104.336998) (width 0.25) (layer F.Cu) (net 1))
 (segment (start 194.31 96.56) (end 190.50999 100.36001) (width 0.25) (layer F.Cu) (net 1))
 (segment (start 190.50999 100.36001) (end 190.50999 103.076988) (width 0.25) (layer F.Cu) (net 1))
 (segment (start 191.77 104.336998) (end 191.77 105.41) (width 0.25) (layer F.Cu) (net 1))
 (segment (start 187.325 102.51) (end 187.325 101.535) (width 0.25) (layer F.Cu) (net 1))
 (segment (start 190.225 105.41) (end 187.325 102.51) (width 0.25) (layer F.Cu) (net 1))
 (segment (start 191.77 105.41) (end 190.225 105.41) (width 0.25) (layer F.Cu) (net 1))
 (segment (start 188.595 102.51) (end 188.595 101.535) (width 0.25) (layer F.Cu) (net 2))
 (segment (start 188.895 101.235) (end 188.595 101.535) (width 0.25) (layer F.Cu) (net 2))
 (segment (start 193.184999 95.685001) (end 193.184999 96.568233) (width 0.25) (layer F.Cu) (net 2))
 (segment (start 188.895 100.858232) (end 188.895 101.235) (width 0.25) (layer F.Cu) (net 2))
 (segment (start 193.184999 96.568233) (end 188.895 100.858232) (width 0.25) (layer F.Cu) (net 2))
 (segment (start 194.31 94.56) (end 193.184999 95.685001) (width 0.25) (layer F.Cu) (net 2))
 (segment (start 156.065001 100.474999) (end 157.335001 100.474999) (width 0.25) (layer B.Cu) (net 5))
 (segment (start 160.490001 97.319999) (end 161.29 96.52) (width 0.25) (layer B.Cu) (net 5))
 (segment (start 157.335001 100.474999) (end 160.490001 97.319999) (width 0.25) (layer B.Cu) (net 5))
 (segment (start 154.94 101.6) (end 156.065001 100.474999) (width 0.25) (layer B.Cu) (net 5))
 (segment (start 161.29 93.98) (end 166.37 88.9) (width 0.25) (layer B.Cu) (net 5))
 (segment (start 161.29 96.52) (end 161.29 93.98) (width 0.25) (layer B.Cu) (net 5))
 (segment (start 154.140001 100.800001) (end 154.94 101.6) (width 0.25) (layer B.Cu) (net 5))
 (segment (start 151.274999 97.934999) (end 154.140001 100.800001) (width 0.25) (layer B.Cu) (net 5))
 (segment (start 135.745001 97.934999) (end 151.274999 97.934999) (width 0.25) (layer B.Cu) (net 5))
 (segment (start 134.62 99.06) (end 135.745001 97.934999) (width 0.25) (layer B.Cu) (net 5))
 (segment (start 194.31 92.06) (end 191.445 94.925) (width 0.25) (layer B.Cu) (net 5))
 (via (at 191.445 94.925) (size 0.8) (drill 0.4) (layers F.Cu B.Cu) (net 5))
 (segment (start 191.135 95.235) (end 191.445 94.925) (width 0.25) (layer F.Cu) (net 5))
 (segment (start 191.135 96.585) (end 191.135 95.235) (width 0.25) (layer F.Cu) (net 5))
 (segment (start 167.169999 89.699999) (end 166.37 88.9) (width 0.25) (layer B.Cu) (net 5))
 (segment (start 191.045001 94.525001) (end 171.995001 94.525001) (width 0.25) (layer B.Cu) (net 5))
 (segment (start 171.995001 94.525001) (end 167.169999 89.699999) (width 0.25) (layer B.Cu) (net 5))
 (segment (start 191.445 94.925) (end 191.045001 94.525001) (width 0.25) (layer B.Cu) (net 5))
 (segment (start 189.865 96.585) (end 189.865 95.61) (width 0.25) (layer F.Cu) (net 6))
 (segment (start 189.865 96.585) (end 189.865 97.56) (width 0.25) (layer F.Cu) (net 6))
 (segment (start 148.59 97.65137) (end 148.59 96.52) (width 0.25) (layer F.Cu) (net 6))
 (segment (start 153.663631 102.725001) (end 148.59 97.65137) (width 0.25) (layer F.Cu) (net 6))
 (segment (start 184.101767 102.725001) (end 153.663631 102.725001) (width 0.25) (layer F.Cu) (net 6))
 (segment (start 189.565 97.261768) (end 184.101767 102.725001) (width 0.25) (layer F.Cu) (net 6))
 (segment (start 189.565 96.885) (end 189.565 97.261768) (width 0.25) (layer F.Cu) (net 6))
 (segment (start 189.865 96.585) (end 189.565 96.885) (width 0.25) (layer F.Cu) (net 6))
 (segment (start 188.595 95.61) (end 188.595 96.585) (width 0.25) (layer F.Cu) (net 7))
 (segment (start 152.255001 95.394999) (end 151.929999 95.720001) (width 0.25) (layer F.Cu) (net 7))
 (segment (start 179.610001 95.394999) (end 152.255001 95.394999) (width 0.25) (layer F.Cu) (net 7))
 (segment (start 182.100012 97.88501) (end 179.610001 95.394999) (width 0.25) (layer F.Cu) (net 7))
 (segment (start 151.929999 95.720001) (end 151.13 96.52) (width 0.25) (layer F.Cu) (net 7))
 (segment (start 188.26999 97.88501) (end 182.100012 97.88501) (width 0.25) (layer F.Cu) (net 7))
 (segment (start 188.595 97.56) (end 188.26999 97.88501) (width 0.25) (layer F.Cu) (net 7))
 (segment (start 188.595 96.585) (end 188.595 97.56) (width 0.25) (layer F.Cu) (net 7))
 (segment (start 147.790001 89.699999) (end 148.59 88.9) (width 0.25) (layer F.Cu) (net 28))
 (segment (start 144.924999 92.565001) (end 147.790001 89.699999) (width 0.25) (layer F.Cu) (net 28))
 (segment (start 135.745001 92.565001) (end 144.924999 92.565001) (width 0.25) (layer F.Cu) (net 28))
 (segment (start 134.62 91.44) (end 135.745001 92.565001) (width 0.25) (layer F.Cu) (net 28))
 (segment (start 144.91863 88.9) (end 146.05 88.9) (width 0.25) (layer F.Cu) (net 30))
 (segment (start 135.494998 88.9) (end 144.91863 88.9) (width 0.25) (layer F.Cu) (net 30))
 (segment (start 133.494999 90.899999) (end 135.494998 88.9) (width 0.25) (layer F.Cu) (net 30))
 (segment (start 133.494999 92.854999) (end 133.494999 90.899999) (width 0.25) (layer F.Cu) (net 30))
 (segment (start 134.62 93.98) (end 133.494999 92.854999) (width 0.25) (layer F.Cu) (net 30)))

